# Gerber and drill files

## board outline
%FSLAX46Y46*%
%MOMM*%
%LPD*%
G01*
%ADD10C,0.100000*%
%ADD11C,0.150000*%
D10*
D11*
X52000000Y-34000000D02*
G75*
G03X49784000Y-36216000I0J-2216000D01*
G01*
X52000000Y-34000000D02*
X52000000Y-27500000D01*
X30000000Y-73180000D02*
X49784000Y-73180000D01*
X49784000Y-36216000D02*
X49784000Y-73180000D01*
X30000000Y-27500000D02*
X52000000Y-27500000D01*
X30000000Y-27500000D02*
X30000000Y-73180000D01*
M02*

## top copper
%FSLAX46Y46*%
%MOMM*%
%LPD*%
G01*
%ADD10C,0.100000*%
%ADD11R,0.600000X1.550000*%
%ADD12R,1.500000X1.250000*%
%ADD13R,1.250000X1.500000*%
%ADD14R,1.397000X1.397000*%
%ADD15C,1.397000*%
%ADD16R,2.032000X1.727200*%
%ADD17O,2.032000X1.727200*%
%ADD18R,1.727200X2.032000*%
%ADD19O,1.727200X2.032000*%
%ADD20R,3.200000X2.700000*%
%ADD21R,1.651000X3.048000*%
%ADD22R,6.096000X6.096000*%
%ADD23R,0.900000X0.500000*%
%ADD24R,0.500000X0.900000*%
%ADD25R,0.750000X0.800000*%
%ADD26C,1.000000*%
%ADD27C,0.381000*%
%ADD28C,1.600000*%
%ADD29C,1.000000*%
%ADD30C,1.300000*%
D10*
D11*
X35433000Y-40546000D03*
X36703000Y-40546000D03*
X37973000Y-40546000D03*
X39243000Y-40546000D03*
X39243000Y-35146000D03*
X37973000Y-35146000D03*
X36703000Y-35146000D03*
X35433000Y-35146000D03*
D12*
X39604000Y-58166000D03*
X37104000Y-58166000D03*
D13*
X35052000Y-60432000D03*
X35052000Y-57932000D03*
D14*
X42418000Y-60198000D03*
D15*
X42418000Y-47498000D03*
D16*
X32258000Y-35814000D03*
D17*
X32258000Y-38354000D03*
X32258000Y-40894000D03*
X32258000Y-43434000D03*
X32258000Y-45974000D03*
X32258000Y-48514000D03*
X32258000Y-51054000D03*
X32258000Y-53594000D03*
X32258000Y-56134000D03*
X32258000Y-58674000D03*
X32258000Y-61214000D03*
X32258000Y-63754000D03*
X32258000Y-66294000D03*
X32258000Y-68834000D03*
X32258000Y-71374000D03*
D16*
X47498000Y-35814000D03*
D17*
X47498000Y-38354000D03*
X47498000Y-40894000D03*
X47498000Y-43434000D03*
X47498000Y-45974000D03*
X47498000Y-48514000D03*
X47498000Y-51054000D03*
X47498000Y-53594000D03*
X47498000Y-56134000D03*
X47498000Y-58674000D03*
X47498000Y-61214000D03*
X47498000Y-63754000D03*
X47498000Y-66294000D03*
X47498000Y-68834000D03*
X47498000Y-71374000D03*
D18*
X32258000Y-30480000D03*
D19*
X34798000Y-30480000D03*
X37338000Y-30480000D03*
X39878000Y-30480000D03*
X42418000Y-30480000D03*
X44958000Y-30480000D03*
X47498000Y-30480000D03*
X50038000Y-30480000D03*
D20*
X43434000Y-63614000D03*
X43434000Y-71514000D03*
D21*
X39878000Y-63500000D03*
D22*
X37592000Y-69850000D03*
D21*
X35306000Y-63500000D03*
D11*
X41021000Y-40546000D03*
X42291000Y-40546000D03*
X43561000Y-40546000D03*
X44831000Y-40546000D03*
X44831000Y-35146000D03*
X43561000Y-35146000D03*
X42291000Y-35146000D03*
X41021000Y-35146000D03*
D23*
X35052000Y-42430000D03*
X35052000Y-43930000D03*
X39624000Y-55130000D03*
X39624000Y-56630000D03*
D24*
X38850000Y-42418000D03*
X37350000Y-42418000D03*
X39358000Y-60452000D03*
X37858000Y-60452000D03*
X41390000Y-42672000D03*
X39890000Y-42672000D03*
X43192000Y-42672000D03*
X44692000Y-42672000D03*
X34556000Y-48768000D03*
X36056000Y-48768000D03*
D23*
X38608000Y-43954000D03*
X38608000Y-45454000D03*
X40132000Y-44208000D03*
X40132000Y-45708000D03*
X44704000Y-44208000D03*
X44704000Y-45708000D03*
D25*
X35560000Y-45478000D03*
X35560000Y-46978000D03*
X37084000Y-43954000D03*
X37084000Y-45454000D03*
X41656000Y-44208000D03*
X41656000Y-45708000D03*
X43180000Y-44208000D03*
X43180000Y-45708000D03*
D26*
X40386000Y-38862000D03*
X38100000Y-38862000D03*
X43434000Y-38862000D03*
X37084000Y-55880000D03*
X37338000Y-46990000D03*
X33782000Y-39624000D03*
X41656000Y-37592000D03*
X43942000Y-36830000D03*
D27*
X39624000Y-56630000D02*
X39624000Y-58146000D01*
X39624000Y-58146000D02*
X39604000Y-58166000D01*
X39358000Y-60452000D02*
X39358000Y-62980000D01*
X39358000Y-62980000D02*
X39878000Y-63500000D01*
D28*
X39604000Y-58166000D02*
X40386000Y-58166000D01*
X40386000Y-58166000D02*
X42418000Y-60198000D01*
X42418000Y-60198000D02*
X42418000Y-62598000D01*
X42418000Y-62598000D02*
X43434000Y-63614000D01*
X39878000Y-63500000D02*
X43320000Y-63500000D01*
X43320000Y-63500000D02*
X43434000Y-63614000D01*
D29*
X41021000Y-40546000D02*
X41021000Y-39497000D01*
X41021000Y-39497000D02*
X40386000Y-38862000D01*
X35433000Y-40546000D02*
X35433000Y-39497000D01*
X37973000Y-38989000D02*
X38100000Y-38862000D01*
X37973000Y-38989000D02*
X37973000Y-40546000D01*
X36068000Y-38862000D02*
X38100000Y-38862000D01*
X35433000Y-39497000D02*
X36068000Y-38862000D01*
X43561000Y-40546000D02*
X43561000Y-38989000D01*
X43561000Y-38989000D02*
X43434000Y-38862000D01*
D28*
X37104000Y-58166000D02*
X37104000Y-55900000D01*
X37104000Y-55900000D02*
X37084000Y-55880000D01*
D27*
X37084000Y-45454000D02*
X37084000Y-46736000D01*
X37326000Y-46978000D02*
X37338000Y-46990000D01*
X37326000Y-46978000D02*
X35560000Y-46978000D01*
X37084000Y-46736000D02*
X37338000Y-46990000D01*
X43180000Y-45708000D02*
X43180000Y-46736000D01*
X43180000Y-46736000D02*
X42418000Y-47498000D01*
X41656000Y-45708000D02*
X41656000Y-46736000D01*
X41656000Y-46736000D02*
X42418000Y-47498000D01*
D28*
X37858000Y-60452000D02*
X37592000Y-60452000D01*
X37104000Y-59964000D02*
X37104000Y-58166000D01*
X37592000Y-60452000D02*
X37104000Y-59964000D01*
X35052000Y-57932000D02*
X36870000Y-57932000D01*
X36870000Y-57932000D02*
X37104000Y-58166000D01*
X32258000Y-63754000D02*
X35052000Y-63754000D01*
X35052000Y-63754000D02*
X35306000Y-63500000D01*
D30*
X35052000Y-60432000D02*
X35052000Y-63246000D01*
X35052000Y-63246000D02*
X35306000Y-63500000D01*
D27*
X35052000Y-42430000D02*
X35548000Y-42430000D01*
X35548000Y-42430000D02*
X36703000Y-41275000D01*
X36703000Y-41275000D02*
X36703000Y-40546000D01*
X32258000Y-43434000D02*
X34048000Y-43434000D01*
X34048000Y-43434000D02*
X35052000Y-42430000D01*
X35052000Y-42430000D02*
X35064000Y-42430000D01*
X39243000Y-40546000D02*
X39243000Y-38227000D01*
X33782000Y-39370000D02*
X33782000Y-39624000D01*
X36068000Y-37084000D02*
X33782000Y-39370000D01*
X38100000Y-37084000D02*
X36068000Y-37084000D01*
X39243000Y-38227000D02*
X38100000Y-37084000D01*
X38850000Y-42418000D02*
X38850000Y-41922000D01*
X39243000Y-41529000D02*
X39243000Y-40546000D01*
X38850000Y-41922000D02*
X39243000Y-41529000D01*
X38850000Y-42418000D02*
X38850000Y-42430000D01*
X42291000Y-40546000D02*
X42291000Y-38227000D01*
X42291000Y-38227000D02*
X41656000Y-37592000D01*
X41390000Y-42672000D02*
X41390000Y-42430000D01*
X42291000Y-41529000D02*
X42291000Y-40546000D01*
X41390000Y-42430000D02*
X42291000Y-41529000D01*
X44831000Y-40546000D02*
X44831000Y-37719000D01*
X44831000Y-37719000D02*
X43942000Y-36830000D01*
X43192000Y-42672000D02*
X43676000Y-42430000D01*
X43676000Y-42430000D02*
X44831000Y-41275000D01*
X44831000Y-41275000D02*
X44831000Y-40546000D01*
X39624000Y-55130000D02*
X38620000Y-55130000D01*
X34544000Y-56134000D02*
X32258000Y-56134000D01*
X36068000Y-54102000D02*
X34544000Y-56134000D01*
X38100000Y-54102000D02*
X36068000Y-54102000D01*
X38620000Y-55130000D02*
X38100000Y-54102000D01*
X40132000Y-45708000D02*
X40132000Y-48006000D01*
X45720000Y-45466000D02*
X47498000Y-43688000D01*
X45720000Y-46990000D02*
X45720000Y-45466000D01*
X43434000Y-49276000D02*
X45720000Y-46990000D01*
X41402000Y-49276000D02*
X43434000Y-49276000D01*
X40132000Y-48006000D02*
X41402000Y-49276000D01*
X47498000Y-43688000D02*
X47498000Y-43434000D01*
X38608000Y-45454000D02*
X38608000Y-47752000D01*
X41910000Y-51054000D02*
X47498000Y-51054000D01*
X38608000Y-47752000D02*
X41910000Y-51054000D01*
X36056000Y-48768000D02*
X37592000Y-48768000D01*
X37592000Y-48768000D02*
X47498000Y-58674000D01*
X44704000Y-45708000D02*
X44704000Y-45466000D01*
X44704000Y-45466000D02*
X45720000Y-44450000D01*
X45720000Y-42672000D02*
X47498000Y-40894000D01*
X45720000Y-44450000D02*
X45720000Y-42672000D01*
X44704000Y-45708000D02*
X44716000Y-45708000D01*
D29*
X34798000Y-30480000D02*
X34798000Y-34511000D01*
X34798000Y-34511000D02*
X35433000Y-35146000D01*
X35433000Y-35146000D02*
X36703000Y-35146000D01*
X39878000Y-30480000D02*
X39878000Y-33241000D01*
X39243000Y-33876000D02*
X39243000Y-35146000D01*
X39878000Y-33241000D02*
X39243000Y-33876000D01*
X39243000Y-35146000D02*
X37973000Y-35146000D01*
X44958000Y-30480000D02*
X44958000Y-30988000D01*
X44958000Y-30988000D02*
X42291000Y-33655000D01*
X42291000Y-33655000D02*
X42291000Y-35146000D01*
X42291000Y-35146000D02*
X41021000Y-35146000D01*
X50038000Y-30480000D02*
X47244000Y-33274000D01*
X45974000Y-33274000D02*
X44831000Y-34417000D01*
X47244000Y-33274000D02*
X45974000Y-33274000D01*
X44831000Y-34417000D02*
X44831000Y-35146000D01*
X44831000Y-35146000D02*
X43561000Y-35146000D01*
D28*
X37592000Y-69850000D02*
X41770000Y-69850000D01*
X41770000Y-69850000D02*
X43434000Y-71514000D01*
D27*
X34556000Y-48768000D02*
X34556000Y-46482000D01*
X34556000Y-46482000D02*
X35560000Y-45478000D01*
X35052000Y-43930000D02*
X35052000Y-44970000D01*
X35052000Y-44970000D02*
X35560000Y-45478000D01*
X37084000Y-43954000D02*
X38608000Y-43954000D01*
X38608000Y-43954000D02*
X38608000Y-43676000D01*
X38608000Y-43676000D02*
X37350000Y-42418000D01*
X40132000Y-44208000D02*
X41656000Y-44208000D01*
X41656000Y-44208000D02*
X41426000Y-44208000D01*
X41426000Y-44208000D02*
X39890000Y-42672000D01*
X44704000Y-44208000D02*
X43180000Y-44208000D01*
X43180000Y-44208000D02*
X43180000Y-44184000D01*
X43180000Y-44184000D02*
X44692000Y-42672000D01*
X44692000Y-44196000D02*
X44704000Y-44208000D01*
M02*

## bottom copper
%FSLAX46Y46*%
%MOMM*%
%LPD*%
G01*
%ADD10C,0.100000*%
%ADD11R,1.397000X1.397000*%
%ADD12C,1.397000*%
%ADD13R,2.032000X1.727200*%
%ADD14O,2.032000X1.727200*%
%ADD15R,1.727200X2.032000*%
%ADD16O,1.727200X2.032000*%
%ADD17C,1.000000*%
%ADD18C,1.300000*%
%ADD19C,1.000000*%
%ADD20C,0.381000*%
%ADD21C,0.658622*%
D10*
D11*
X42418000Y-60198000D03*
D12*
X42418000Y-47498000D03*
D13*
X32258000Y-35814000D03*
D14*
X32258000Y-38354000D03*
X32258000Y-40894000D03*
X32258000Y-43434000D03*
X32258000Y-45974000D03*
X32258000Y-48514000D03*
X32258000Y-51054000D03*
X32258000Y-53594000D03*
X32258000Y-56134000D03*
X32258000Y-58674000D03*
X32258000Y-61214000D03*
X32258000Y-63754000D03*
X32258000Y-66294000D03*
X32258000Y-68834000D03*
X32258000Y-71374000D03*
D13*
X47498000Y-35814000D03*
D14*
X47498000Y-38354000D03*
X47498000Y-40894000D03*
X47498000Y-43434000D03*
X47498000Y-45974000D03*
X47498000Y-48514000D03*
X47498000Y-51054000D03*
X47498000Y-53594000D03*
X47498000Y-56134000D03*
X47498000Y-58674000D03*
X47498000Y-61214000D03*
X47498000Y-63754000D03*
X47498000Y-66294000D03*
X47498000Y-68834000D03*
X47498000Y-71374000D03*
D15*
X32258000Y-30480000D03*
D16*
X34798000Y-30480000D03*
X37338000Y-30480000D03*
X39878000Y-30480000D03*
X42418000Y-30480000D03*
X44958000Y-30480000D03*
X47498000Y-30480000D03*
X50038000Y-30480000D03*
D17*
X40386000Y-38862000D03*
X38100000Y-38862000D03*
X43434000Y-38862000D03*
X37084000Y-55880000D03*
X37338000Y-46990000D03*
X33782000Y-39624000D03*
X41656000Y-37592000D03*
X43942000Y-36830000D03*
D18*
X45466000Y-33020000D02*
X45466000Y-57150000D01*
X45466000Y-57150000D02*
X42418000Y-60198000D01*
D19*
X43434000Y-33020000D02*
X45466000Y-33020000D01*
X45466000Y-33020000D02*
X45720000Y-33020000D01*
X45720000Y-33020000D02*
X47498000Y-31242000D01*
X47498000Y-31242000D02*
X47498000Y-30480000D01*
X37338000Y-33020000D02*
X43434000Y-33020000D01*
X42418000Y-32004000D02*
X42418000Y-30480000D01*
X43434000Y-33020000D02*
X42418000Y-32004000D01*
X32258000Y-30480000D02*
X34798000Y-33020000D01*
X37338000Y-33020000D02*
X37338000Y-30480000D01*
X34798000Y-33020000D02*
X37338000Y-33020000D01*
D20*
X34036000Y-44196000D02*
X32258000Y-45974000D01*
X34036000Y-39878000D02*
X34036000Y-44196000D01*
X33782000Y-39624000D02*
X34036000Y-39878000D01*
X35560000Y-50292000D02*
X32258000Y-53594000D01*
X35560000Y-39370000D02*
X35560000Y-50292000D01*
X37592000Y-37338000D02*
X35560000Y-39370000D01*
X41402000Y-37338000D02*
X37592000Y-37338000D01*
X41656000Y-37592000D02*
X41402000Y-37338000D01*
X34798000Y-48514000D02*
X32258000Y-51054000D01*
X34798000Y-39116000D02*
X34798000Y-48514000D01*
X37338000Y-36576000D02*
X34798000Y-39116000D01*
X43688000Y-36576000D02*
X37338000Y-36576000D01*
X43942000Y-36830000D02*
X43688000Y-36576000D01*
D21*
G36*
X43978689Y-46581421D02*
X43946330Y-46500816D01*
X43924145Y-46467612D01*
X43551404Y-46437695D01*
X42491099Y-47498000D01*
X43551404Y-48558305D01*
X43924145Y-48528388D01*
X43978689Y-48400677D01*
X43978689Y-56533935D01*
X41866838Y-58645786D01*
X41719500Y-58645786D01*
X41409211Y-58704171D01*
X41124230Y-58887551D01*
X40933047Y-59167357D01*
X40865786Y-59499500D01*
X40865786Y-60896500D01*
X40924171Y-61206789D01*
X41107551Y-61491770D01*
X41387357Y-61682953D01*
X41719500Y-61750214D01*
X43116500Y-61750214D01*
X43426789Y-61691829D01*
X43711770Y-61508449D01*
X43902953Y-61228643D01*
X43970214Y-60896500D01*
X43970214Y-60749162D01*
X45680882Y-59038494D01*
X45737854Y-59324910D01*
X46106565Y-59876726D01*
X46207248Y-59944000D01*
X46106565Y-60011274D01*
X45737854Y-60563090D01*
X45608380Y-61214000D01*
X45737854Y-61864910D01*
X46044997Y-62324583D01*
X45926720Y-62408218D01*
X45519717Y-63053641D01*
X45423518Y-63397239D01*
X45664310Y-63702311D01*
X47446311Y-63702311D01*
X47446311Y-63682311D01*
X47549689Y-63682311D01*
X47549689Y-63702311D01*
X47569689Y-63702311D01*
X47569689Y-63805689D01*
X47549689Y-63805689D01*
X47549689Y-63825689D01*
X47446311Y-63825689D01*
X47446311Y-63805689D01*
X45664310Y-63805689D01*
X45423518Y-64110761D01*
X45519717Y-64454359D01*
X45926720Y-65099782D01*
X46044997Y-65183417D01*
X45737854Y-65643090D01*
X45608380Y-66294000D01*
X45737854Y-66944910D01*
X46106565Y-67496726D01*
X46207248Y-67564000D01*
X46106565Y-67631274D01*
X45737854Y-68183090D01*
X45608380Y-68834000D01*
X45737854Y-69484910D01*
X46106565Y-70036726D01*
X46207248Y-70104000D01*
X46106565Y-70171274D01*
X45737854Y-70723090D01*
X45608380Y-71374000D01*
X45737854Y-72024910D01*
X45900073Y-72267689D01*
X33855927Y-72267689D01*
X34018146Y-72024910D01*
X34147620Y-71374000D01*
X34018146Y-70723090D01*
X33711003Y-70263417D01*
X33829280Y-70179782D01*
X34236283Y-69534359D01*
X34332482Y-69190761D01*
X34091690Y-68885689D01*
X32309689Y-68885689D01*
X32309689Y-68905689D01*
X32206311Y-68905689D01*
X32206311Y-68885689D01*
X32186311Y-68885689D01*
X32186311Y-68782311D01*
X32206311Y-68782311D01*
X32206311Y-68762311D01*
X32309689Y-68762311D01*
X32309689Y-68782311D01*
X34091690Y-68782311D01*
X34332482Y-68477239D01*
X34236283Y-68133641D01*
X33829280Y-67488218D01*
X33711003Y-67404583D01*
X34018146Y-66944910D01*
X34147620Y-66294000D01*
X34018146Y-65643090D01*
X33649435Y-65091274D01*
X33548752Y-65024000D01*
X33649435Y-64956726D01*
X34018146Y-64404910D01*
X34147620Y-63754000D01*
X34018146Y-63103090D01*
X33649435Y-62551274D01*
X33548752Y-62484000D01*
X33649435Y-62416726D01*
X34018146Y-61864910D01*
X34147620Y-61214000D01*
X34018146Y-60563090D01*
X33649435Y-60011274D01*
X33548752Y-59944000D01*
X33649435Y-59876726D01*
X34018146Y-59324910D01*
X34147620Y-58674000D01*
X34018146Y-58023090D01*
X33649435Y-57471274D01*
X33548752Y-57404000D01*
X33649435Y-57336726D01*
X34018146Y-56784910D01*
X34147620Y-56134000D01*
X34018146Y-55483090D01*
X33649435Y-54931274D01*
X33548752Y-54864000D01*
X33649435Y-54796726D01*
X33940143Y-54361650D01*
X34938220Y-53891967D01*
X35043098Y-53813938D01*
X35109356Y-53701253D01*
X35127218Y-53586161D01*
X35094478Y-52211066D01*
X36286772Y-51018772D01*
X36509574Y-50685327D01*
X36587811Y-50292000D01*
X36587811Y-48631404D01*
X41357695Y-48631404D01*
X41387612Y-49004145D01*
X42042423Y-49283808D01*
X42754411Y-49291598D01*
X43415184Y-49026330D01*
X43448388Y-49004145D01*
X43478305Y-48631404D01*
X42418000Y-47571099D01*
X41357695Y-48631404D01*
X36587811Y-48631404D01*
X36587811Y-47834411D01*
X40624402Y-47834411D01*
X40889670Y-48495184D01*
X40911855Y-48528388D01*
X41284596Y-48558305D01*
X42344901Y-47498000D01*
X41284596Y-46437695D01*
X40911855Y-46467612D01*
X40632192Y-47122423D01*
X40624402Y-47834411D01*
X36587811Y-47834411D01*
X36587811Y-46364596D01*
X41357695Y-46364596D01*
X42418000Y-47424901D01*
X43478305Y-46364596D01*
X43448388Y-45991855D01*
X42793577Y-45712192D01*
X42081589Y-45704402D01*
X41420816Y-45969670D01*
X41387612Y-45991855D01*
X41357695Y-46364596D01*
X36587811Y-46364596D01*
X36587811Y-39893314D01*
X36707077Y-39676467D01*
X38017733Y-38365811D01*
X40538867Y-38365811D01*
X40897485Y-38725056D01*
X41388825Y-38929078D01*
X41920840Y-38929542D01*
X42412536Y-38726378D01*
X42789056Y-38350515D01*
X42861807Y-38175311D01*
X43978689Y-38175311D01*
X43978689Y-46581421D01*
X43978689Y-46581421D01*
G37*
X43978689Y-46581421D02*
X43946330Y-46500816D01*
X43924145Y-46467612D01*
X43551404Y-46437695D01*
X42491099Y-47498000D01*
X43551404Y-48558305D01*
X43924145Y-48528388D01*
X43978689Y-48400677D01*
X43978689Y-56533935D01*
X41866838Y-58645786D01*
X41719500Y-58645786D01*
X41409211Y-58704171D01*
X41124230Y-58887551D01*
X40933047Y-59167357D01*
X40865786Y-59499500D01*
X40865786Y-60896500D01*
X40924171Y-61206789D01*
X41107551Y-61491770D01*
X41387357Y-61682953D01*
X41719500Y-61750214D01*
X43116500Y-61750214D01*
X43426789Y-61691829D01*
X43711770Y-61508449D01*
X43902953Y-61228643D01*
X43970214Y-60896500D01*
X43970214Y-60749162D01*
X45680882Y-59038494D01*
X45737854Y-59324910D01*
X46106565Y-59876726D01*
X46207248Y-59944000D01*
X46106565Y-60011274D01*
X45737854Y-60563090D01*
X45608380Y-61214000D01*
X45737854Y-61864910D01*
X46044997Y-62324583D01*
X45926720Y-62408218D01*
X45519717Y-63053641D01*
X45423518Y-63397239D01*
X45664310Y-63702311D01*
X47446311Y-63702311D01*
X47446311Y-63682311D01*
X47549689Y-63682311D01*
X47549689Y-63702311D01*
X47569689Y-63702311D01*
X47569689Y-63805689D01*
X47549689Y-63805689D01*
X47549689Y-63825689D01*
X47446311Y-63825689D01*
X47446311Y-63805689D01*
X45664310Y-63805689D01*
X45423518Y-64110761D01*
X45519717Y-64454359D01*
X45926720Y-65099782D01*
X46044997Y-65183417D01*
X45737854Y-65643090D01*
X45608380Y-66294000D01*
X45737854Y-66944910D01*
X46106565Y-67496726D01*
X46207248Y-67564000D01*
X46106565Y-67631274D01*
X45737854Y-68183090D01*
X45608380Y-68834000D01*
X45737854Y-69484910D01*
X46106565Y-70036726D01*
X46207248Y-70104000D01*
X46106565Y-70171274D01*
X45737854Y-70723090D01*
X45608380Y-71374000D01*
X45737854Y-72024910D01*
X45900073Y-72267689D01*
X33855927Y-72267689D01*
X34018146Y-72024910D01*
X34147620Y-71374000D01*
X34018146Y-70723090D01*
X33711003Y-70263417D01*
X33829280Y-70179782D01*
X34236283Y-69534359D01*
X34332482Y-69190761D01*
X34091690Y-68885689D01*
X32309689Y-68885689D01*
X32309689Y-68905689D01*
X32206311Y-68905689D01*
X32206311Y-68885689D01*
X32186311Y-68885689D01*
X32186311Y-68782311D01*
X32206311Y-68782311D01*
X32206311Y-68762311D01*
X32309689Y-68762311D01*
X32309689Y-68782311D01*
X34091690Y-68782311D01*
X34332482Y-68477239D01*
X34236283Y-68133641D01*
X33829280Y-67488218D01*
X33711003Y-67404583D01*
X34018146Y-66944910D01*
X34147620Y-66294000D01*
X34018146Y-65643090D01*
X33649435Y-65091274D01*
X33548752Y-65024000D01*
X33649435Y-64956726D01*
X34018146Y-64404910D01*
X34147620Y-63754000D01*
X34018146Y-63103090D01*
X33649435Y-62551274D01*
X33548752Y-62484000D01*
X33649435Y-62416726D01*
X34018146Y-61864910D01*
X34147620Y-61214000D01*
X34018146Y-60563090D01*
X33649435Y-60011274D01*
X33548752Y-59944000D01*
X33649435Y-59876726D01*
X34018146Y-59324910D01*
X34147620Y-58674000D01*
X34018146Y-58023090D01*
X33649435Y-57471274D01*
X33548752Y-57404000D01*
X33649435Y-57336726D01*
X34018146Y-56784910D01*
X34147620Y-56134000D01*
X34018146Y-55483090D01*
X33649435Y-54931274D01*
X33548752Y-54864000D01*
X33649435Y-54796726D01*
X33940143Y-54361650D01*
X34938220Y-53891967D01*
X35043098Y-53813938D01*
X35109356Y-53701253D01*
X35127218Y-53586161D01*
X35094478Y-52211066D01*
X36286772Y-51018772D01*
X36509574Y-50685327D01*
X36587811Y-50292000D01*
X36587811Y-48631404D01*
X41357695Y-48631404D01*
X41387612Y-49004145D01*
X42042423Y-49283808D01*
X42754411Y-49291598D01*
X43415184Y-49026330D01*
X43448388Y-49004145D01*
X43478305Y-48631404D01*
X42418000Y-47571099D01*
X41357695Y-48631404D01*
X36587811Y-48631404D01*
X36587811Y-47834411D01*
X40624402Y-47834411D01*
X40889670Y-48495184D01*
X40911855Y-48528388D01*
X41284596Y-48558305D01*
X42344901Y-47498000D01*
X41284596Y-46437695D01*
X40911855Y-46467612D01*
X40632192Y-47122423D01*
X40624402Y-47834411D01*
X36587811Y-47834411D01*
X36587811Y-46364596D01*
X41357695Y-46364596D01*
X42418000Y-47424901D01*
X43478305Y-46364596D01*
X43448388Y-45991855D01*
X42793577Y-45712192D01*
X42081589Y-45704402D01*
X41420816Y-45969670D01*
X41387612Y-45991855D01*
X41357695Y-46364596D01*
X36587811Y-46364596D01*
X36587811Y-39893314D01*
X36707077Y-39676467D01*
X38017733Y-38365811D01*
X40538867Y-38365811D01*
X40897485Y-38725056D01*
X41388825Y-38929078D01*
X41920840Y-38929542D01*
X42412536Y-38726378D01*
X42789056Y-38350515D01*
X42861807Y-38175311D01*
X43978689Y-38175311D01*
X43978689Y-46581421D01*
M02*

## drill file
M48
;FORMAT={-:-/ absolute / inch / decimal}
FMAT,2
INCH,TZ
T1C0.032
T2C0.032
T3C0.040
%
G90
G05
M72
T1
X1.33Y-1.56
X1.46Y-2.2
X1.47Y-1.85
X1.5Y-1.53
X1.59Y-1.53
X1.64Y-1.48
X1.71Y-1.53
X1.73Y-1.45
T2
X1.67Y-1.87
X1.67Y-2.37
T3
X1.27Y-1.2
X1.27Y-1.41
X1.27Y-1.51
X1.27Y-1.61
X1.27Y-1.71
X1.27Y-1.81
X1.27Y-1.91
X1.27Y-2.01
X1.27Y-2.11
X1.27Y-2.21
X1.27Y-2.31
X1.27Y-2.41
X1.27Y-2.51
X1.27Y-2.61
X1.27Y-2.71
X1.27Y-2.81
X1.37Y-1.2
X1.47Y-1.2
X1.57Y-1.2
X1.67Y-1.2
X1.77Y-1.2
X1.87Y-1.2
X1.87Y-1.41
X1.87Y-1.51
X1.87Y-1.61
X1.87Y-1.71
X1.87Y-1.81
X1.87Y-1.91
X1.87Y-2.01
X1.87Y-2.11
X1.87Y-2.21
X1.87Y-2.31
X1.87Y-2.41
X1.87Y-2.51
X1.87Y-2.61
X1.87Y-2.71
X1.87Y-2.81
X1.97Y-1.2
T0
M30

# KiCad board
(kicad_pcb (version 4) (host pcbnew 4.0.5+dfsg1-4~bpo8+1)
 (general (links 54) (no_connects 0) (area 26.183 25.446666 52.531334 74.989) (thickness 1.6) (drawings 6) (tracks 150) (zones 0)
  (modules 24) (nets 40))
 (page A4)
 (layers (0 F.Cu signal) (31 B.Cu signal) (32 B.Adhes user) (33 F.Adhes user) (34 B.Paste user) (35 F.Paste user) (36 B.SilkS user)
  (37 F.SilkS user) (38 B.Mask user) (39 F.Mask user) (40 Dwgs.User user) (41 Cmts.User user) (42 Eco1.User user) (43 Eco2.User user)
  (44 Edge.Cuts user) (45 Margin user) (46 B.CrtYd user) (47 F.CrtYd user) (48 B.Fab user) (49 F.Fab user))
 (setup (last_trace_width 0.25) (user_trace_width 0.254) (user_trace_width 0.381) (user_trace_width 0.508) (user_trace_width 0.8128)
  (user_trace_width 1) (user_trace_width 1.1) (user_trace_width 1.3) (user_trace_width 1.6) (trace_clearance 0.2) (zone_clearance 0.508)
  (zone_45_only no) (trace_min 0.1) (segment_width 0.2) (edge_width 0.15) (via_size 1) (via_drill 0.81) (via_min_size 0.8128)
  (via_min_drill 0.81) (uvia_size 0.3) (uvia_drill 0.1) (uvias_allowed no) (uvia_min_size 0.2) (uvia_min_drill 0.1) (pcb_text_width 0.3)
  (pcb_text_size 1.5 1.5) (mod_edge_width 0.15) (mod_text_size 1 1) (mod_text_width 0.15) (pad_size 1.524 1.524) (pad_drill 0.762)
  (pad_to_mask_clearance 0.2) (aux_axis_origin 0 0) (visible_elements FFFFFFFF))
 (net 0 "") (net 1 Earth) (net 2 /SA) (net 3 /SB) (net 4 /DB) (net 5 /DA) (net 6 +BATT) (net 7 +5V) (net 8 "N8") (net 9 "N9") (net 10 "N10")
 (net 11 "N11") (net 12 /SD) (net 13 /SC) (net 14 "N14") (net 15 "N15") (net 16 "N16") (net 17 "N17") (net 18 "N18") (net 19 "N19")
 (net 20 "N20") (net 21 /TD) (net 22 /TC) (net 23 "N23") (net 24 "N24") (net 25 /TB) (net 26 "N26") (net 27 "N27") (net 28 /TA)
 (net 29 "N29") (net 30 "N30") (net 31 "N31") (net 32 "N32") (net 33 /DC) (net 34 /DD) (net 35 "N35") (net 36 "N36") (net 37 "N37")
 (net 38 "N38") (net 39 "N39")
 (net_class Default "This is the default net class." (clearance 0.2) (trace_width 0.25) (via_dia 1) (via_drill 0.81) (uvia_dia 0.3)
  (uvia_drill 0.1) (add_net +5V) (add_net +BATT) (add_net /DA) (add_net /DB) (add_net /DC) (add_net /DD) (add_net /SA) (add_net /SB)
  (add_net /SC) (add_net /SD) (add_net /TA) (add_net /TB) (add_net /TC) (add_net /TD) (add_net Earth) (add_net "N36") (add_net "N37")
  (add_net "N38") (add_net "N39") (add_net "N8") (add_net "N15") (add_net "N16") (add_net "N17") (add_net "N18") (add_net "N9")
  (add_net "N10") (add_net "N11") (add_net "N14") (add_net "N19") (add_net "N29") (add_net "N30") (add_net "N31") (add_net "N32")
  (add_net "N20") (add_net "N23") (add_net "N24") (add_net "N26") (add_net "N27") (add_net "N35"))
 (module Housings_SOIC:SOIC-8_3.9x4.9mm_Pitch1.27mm (layer F.Cu) (at 37.338 37.846 90)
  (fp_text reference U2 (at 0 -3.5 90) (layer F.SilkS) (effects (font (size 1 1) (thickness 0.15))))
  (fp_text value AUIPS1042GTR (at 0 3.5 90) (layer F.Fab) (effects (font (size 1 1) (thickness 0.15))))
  (pad 1 smd rect (at -2.7 -1.905 90) (size 1.55 0.6) (layers F.Cu F.Paste F.Mask) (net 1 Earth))
  (pad 2 smd rect (at -2.7 -0.635 90) (size 1.55 0.6) (layers F.Cu F.Paste F.Mask) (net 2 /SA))
  (pad 3 smd rect (at -2.7 0.635 90) (size 1.55 0.6) (layers F.Cu F.Paste F.Mask) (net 1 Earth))
  (pad 4 smd rect (at -2.7 1.905 90) (size 1.55 0.6) (layers F.Cu F.Paste F.Mask) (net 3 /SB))
  (pad 5 smd rect (at 2.7 1.905 90) (size 1.55 0.6) (layers F.Cu F.Paste F.Mask) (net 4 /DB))
  (pad 6 smd rect (at 2.7 0.635 90) (size 1.55 0.6) (layers F.Cu F.Paste F.Mask) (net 4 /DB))
  (pad 7 smd rect (at 2.7 -0.635 90) (size 1.55 0.6) (layers F.Cu F.Paste F.Mask) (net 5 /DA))
  (pad 8 smd rect (at 2.7 -1.905 90) (size 1.55 0.6) (layers F.Cu F.Paste F.Mask) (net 5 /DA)))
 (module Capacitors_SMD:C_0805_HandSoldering (layer F.Cu) (at 38.354 58.166 180)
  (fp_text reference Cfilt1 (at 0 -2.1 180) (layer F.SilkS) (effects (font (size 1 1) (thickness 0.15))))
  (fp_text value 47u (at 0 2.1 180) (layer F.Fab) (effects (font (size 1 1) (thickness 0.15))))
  (pad 1 smd rect (at -1.25 0 180) (size 1.5 1.25) (layers F.Cu F.Paste F.Mask) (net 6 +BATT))
  (pad 2 smd rect (at 1.25 0 180) (size 1.5 1.25) (layers F.Cu F.Paste F.Mask) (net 1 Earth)))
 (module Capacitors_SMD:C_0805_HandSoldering (layer F.Cu) (at 35.052 59.182 90)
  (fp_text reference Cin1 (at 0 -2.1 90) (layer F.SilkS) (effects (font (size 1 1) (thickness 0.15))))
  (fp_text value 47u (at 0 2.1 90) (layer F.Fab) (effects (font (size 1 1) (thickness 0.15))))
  (pad 1 smd rect (at -1.25 0 90) (size 1.5 1.25) (layers F.Cu F.Paste F.Mask) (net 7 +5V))
  (pad 2 smd rect (at 1.25 0 90) (size 1.5 1.25) (layers F.Cu F.Paste F.Mask) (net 1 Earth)))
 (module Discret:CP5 (layer F.Cu) (at 42.418 53.848 90)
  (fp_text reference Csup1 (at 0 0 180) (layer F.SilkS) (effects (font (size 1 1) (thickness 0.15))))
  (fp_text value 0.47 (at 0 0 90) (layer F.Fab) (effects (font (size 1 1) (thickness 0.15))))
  (pad 1 thru_hole rect (at -6.35 0 90) (size 1.397 1.397) (drill 0.8128) (layers *.Cu *.Mask) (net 6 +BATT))
  (pad 2 thru_hole circle (at 6.35 0 90) (size 1.397 1.397) (drill 0.8128) (layers *.Cu *.Mask) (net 1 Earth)))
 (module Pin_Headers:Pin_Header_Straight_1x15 (layer F.Cu) (at 32.258 35.814)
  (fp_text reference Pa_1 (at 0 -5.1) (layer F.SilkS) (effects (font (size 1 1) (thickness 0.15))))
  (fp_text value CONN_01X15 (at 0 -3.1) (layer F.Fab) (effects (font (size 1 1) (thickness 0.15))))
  (pad 1 thru_hole rect (at 0 0) (size 2.032 1.7272) (drill 1.016) (layers *.Cu *.Mask) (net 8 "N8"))
  (pad 2 thru_hole oval (at 0 2.54) (size 2.032 1.7272) (drill 1.016) (layers *.Cu *.Mask) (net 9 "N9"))
  (pad 3 thru_hole oval (at 0 5.08) (size 2.032 1.7272) (drill 1.016) (layers *.Cu *.Mask) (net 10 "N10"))
  (pad 4 thru_hole oval (at 0 7.62) (size 2.032 1.7272) (drill 1.016) (layers *.Cu *.Mask) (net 2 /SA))
  (pad 5 thru_hole oval (at 0 10.16) (size 2.032 1.7272) (drill 1.016) (layers *.Cu *.Mask) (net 3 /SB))
  (pad 6 thru_hole oval (at 0 12.7) (size 2.032 1.7272) (drill 1.016) (layers *.Cu *.Mask) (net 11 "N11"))
  (pad 7 thru_hole oval (at 0 15.24) (size 2.032 1.7272) (drill 1.016) (layers *.Cu *.Mask) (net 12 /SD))
  (pad 8 thru_hole oval (at 0 17.78) (size 2.032 1.7272) (drill 1.016) (layers *.Cu *.Mask) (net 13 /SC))
  (pad 9 thru_hole oval (at 0 20.32) (size 2.032 1.7272) (drill 1.016) (layers *.Cu *.Mask) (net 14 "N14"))
  (pad 10 thru_hole oval (at 0 22.86) (size 2.032 1.7272) (drill 1.016) (layers *.Cu *.Mask) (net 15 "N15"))
  (pad 11 thru_hole oval (at 0 25.4) (size 2.032 1.7272) (drill 1.016) (layers *.Cu *.Mask) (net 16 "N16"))
  (pad 12 thru_hole oval (at 0 27.94) (size 2.032 1.7272) (drill 1.016) (layers *.Cu *.Mask) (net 7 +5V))
  (pad 13 thru_hole oval (at 0 30.48) (size 2.032 1.7272) (drill 1.016) (layers *.Cu *.Mask) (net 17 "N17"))
  (pad 14 thru_hole oval (at 0 33.02) (size 2.032 1.7272) (drill 1.016) (layers *.Cu *.Mask) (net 1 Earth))
  (pad 15 thru_hole oval (at 0 35.56) (size 2.032 1.7272) (drill 1.016) (layers *.Cu *.Mask) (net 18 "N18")))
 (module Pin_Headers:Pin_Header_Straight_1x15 (layer F.Cu) (at 47.498 35.814)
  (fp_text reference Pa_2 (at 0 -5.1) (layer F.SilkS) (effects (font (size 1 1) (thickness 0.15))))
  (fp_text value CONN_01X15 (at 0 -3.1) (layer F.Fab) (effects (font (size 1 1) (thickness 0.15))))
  (pad 1 thru_hole rect (at 0 0) (size 2.032 1.7272) (drill 1.016) (layers *.Cu *.Mask) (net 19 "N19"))
  (pad 2 thru_hole oval (at 0 2.54) (size 2.032 1.7272) (drill 1.016) (layers *.Cu *.Mask) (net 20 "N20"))
  (pad 3 thru_hole oval (at 0 5.08) (size 2.032 1.7272) (drill 1.016) (layers *.Cu *.Mask) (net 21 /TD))
  (pad 4 thru_hole oval (at 0 7.62) (size 2.032 1.7272) (drill 1.016) (layers *.Cu *.Mask) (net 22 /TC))
  (pad 5 thru_hole oval (at 0 10.16) (size 2.032 1.7272) (drill 1.016) (layers *.Cu *.Mask) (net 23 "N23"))
  (pad 6 thru_hole oval (at 0 12.7) (size 2.032 1.7272) (drill 1.016) (layers *.Cu *.Mask) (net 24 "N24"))
  (pad 7 thru_hole oval (at 0 15.24) (size 2.032 1.7272) (drill 1.016) (layers *.Cu *.Mask) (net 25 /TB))
  (pad 8 thru_hole oval (at 0 17.78) (size 2.032 1.7272) (drill 1.016) (layers *.Cu *.Mask) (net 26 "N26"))
  (pad 9 thru_hole oval (at 0 20.32) (size 2.032 1.7272) (drill 1.016) (layers *.Cu *.Mask) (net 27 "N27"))
  (pad 10 thru_hole oval (at 0 22.86) (size 2.032 1.7272) (drill 1.016) (layers *.Cu *.Mask) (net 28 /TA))
  (pad 11 thru_hole oval (at 0 25.4) (size 2.032 1.7272) (drill 1.016) (layers *.Cu *.Mask) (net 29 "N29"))
  (pad 12 thru_hole oval (at 0 27.94) (size 2.032 1.7272) (drill 1.016) (layers *.Cu *.Mask) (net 1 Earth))
  (pad 13 thru_hole oval (at 0 30.48) (size 2.032 1.7272) (drill 1.016) (layers *.Cu *.Mask) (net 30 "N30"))
  (pad 14 thru_hole oval (at 0 33.02) (size 2.032 1.7272) (drill 1.016) (layers *.Cu *.Mask) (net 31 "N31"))
  (pad 15 thru_hole oval (at 0 35.56) (size 2.032 1.7272) (drill 1.016) (layers *.Cu *.Mask) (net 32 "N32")))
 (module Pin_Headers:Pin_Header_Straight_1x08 (layer F.Cu) (at 32.258 30.48 90)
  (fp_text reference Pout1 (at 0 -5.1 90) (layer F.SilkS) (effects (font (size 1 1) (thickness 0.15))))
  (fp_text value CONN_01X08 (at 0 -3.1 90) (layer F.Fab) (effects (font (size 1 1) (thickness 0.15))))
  (pad 1 thru_hole rect (at 0 0 90) (size 2.032 1.7272) (drill 1.016) (layers *.Cu *.Mask) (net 6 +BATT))
  (pad 2 thru_hole oval (at 0 2.54 90) (size 2.032 1.7272) (drill 1.016) (layers *.Cu *.Mask) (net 5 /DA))
  (pad 3 thru_hole oval (at 0 5.08 90) (size 2.032 1.7272) (drill 1.016) (layers *.Cu *.Mask) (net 6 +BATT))
  (pad 4 thru_hole oval (at 0 7.62 90) (size 2.032 1.7272) (drill 1.016) (layers *.Cu *.Mask) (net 4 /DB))
  (pad 5 thru_hole oval (at 0 10.16 90) (size 2.032 1.7272) (drill 1.016) (layers *.Cu *.Mask) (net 6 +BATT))
  (pad 6 thru_hole oval (at 0 12.7 90) (size 2.032 1.7272) (drill 1.016) (layers *.Cu *.Mask) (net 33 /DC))
  (pad 7 thru_hole oval (at 0 15.24 90) (size 2.032 1.7272) (drill 1.016) (layers *.Cu *.Mask) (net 6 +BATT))
  (pad 8 thru_hole oval (at 0 17.78 90) (size 2.032 1.7272) (drill 1.016) (layers *.Cu *.Mask) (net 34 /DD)))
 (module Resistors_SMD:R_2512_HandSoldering (layer F.Cu) (at 43.434 67.564 270)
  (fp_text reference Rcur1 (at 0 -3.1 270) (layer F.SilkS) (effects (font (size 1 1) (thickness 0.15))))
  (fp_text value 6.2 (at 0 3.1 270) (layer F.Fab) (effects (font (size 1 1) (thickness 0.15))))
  (pad 1 smd rect (at -3.95 0 270) (size 2.7 3.2) (layers F.Cu F.Paste F.Mask) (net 6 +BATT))
  (pad 2 smd rect (at 3.95 0 270) (size 2.7 3.2) (layers F.Cu F.Paste F.Mask) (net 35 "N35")))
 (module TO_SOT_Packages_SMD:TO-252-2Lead (layer F.Cu) (at 37.592 63.5 180)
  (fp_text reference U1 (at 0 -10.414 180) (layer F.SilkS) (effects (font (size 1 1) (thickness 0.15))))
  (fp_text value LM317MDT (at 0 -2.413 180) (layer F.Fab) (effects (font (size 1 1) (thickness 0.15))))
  (pad 1 smd rect (at -2.286 0 180) (size 1.651 3.048) (layers F.Cu F.Paste F.Mask) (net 6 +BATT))
  (pad 2 smd rect (at 0 -6.35 180) (size 6.096 6.096) (layers F.Cu F.Paste F.Mask) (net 35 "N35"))
  (pad 3 smd rect (at 2.286 0 180) (size 1.651 3.048) (layers F.Cu F.Paste F.Mask) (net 7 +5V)))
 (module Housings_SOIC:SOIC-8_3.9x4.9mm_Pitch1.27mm (layer F.Cu) (at 42.926 37.846 90)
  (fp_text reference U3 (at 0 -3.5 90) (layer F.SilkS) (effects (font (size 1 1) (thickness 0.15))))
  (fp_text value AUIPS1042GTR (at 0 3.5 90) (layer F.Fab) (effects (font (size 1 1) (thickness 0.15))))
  (pad 1 smd rect (at -2.7 -1.905 90) (size 1.55 0.6) (layers F.Cu F.Paste F.Mask) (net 1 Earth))
  (pad 2 smd rect (at -2.7 -0.635 90) (size 1.55 0.6) (layers F.Cu F.Paste F.Mask) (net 13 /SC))
  (pad 3 smd rect (at -2.7 0.635 90) (size 1.55 0.6) (layers F.Cu F.Paste F.Mask) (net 1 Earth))
  (pad 4 smd rect (at -2.7 1.905 90) (size 1.55 0.6) (layers F.Cu F.Paste F.Mask) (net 12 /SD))
  (pad 5 smd rect (at 2.7 1.905 90) (size 1.55 0.6) (layers F.Cu F.Paste F.Mask) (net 34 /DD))
  (pad 6 smd rect (at 2.7 0.635 90) (size 1.55 0.6) (layers F.Cu F.Paste F.Mask) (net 34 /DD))
  (pad 7 smd rect (at 2.7 -0.635 90) (size 1.55 0.6) (layers F.Cu F.Paste F.Mask) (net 33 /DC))
  (pad 8 smd rect (at 2.7 -1.905 90) (size 1.55 0.6) (layers F.Cu F.Paste F.Mask) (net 33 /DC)))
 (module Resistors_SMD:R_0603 (layer F.Cu) (at 35.052 43.18 270)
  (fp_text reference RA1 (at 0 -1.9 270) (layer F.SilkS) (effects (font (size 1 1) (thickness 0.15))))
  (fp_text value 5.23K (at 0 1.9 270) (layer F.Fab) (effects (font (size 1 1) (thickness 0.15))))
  (pad 1 smd rect (at -0.75 0 270) (size 0.5 0.9) (layers F.Cu F.Paste F.Mask) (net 2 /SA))
  (pad 2 smd rect (at 0.75 0 270) (size 0.5 0.9) (layers F.Cu F.Paste F.Mask) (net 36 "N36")))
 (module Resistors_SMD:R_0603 (layer F.Cu) (at 39.624 55.88 270)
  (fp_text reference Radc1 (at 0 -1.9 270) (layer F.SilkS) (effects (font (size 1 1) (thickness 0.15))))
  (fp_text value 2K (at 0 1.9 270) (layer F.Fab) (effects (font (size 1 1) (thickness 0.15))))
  (pad 1 smd rect (at -0.75 0 270) (size 0.5 0.9) (layers F.Cu F.Paste F.Mask) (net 14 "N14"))
  (pad 2 smd rect (at 0.75 0 270) (size 0.5 0.9) (layers F.Cu F.Paste F.Mask) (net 6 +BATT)))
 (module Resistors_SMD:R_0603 (layer F.Cu) (at 38.1 42.418 180)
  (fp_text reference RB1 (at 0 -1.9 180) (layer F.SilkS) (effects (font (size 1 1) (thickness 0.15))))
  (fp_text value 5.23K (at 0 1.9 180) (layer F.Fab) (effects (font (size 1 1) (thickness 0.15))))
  (pad 1 smd rect (at -0.75 0 180) (size 0.5 0.9) (layers F.Cu F.Paste F.Mask) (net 3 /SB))
  (pad 2 smd rect (at 0.75 0 180) (size 0.5 0.9) (layers F.Cu F.Paste F.Mask) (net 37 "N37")))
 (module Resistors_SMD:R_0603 (layer F.Cu) (at 38.608 60.452 180)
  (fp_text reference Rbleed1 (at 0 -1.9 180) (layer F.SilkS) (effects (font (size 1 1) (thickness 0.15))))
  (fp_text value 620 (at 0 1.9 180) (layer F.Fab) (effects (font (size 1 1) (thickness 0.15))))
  (pad 1 smd rect (at -0.75 0 180) (size 0.5 0.9) (layers F.Cu F.Paste F.Mask) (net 6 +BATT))
  (pad 2 smd rect (at 0.75 0 180) (size 0.5 0.9) (layers F.Cu F.Paste F.Mask) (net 1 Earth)))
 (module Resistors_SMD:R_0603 (layer F.Cu) (at 40.64 42.672 180)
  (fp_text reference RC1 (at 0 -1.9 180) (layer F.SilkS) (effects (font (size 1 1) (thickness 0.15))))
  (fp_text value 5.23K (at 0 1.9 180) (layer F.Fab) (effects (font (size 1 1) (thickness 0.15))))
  (pad 1 smd rect (at -0.75 0 180) (size 0.5 0.9) (layers F.Cu F.Paste F.Mask) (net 13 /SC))
  (pad 2 smd rect (at 0.75 0 180) (size 0.5 0.9) (layers F.Cu F.Paste F.Mask) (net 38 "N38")))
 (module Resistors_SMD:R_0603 (layer F.Cu) (at 43.942 42.672)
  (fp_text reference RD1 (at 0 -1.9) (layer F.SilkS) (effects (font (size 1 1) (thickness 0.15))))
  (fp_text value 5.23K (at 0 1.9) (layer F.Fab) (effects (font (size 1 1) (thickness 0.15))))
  (pad 1 smd rect (at -0.75 0) (size 0.5 0.9) (layers F.Cu F.Paste F.Mask) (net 12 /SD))
  (pad 2 smd rect (at 0.75 0) (size 0.5 0.9) (layers F.Cu F.Paste F.Mask) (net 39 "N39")))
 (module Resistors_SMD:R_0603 (layer F.Cu) (at 35.306 48.768)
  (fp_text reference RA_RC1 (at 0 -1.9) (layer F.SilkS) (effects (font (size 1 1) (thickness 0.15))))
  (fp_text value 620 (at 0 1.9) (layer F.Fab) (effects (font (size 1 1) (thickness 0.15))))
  (pad 1 smd rect (at -0.75 0) (size 0.5 0.9) (layers F.Cu F.Paste F.Mask) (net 36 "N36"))
  (pad 2 smd rect (at 0.75 0) (size 0.5 0.9) (layers F.Cu F.Paste F.Mask) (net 28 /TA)))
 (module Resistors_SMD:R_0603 (layer F.Cu) (at 38.608 44.704 270)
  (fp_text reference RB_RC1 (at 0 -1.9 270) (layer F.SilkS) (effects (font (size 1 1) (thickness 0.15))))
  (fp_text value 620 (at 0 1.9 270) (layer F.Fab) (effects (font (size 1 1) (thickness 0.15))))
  (pad 1 smd rect (at -0.75 0 270) (size 0.5 0.9) (layers F.Cu F.Paste F.Mask) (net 37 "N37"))
  (pad 2 smd rect (at 0.75 0 270) (size 0.5 0.9) (layers F.Cu F.Paste F.Mask) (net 25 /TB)))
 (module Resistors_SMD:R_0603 (layer F.Cu) (at 40.132 44.958 270)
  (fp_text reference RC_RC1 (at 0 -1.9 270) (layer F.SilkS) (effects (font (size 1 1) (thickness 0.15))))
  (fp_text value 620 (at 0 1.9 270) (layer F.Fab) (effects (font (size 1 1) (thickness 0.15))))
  (pad 1 smd rect (at -0.75 0 270) (size 0.5 0.9) (layers F.Cu F.Paste F.Mask) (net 38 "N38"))
  (pad 2 smd rect (at 0.75 0 270) (size 0.5 0.9) (layers F.Cu F.Paste F.Mask) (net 22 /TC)))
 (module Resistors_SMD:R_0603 (layer F.Cu) (at 44.704 44.958 270)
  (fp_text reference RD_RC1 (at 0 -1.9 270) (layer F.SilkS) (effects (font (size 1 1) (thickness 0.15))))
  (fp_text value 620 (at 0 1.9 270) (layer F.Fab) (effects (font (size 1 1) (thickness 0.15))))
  (pad 1 smd rect (at -0.75 0 270) (size 0.5 0.9) (layers F.Cu F.Paste F.Mask) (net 39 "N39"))
  (pad 2 smd rect (at 0.75 0 270) (size 0.5 0.9) (layers F.Cu F.Paste F.Mask) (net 21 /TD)))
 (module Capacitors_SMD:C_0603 (layer F.Cu) (at 35.56 46.228 270)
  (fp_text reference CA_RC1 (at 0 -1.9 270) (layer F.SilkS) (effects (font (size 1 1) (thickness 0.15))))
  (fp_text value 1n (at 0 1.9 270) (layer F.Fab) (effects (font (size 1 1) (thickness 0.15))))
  (pad 1 smd rect (at -0.75 0 270) (size 0.8 0.75) (layers F.Cu F.Paste F.Mask) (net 36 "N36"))
  (pad 2 smd rect (at 0.75 0 270) (size 0.8 0.75) (layers F.Cu F.Paste F.Mask) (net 1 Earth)))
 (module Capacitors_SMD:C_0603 (layer F.Cu) (at 37.084 44.704 270)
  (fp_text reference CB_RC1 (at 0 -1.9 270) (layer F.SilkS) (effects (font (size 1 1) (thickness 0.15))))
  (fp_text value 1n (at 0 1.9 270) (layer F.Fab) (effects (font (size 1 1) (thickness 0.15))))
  (pad 1 smd rect (at -0.75 0 270) (size 0.8 0.75) (layers F.Cu F.Paste F.Mask) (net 37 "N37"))
  (pad 2 smd rect (at 0.75 0 270) (size 0.8 0.75) (layers F.Cu F.Paste F.Mask) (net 1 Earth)))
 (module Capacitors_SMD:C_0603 (layer F.Cu) (at 41.656 44.958 270)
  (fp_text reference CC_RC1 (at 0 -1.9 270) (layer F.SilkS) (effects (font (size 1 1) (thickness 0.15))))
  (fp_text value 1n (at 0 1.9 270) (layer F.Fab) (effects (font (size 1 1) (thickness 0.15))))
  (pad 1 smd rect (at -0.75 0 270) (size 0.8 0.75) (layers F.Cu F.Paste F.Mask) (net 38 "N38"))
  (pad 2 smd rect (at 0.75 0 270) (size 0.8 0.75) (layers F.Cu F.Paste F.Mask) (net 1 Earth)))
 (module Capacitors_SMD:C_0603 (layer F.Cu) (at 43.18 44.958 270)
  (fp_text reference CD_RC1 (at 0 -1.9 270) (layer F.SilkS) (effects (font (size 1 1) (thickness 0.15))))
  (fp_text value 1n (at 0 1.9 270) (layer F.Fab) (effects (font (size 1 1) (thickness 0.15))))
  (pad 1 smd rect (at -0.75 0 270) (size 0.8 0.75) (layers F.Cu F.Paste F.Mask) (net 39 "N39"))
  (pad 2 smd rect (at 0.75 0 270) (size 0.8 0.75) (layers F.Cu F.Paste F.Mask) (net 1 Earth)))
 (gr_arc (start 52 36.216) (end 49.784 36.216) (angle 90) (layer Edge.Cuts) (width 0.15))
 (gr_line (start 52 34) (end 52 27.5) (angle 90) (layer Edge.Cuts) (width 0.15))
 (gr_line (start 30 73.18) (end 49.784 73.18) (angle 90) (layer Edge.Cuts) (width 0.15))
 (gr_line (start 49.784 36.216) (end 49.784 73.18) (angle 90) (layer Edge.Cuts) (width 0.15))
 (gr_line (start 30 27.5) (end 52 27.5) (angle 90) (layer Edge.Cuts) (width 0.15))
 (gr_line (start 30 27.5) (end 30 73.18) (angle 90) (layer Edge.Cuts) (width 0.15))
 (segment (start 39.624 56.63) (end 39.624 58.146) (width 0.381) (layer F.Cu) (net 6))
 (segment (start 39.624 58.146) (end 39.604 58.166) (width 0.381) (layer F.Cu) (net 6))
 (segment (start 39.358 60.452) (end 39.358 62.98) (width 0.381) (layer F.Cu) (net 6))
 (segment (start 39.358 62.98) (end 39.878 63.5) (width 0.381) (layer F.Cu) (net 6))
 (segment (start 39.604 58.166) (end 40.386 58.166) (width 1.6) (layer F.Cu) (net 6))
 (segment (start 40.386 58.166) (end 42.418 60.198) (width 1.6) (layer F.Cu) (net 6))
 (segment (start 42.418 60.198) (end 42.418 62.598) (width 1.6) (layer F.Cu) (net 6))
 (segment (start 42.418 62.598) (end 43.434 63.614) (width 1.6) (layer F.Cu) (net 6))
 (segment (start 39.878 63.5) (end 43.32 63.5) (width 1.6) (layer F.Cu) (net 6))
 (segment (start 43.32 63.5) (end 43.434 63.614) (width 1.6) (layer F.Cu) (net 6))
 (segment (start 45.466 33.02) (end 45.466 57.15) (width 1.3) (layer B.Cu) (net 6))
 (segment (start 45.466 57.15) (end 42.418 60.198) (width 1.3) (layer B.Cu) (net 6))
 (segment (start 43.434 33.02) (end 45.466 33.02) (width 1) (layer B.Cu) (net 6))
 (segment (start 45.466 33.02) (end 45.72 33.02) (width 1) (layer B.Cu) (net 6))
 (segment (start 45.72 33.02) (end 47.498 31.242) (width 1) (layer B.Cu) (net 6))
 (segment (start 47.498 31.242) (end 47.498 30.48) (width 1) (layer B.Cu) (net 6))
 (segment (start 37.338 33.02) (end 43.434 33.02) (width 1) (layer B.Cu) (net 6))
 (segment (start 42.418 32.004) (end 42.418 30.48) (width 1) (layer B.Cu) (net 6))
 (segment (start 43.434 33.02) (end 42.418 32.004) (width 1) (layer B.Cu) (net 6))
 (segment (start 32.258 30.48) (end 34.798 33.02) (width 1) (layer B.Cu) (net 6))
 (segment (start 37.338 33.02) (end 37.338 30.48) (width 1) (layer B.Cu) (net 6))
 (segment (start 34.798 33.02) (end 37.338 33.02) (width 1) (layer B.Cu) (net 6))
 (segment (start 41.021 40.546) (end 41.021 39.497) (width 1) (layer F.Cu) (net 1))
 (via (at 40.386 38.862) (size 1) (drill 0.81) (layers F.Cu B.Cu) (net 1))
 (segment (start 41.021 39.497) (end 40.386 38.862) (width 1) (layer F.Cu) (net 1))
 (segment (start 35.433 40.546) (end 35.433 39.497) (width 1) (layer F.Cu) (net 1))
 (segment (start 37.973 38.989) (end 38.1 38.862) (width 1) (layer F.Cu) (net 1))
 (via (at 38.1 38.862) (size 1) (drill 0.81) (layers F.Cu B.Cu) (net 1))
 (segment (start 37.973 38.989) (end 37.973 40.546) (width 1) (layer F.Cu) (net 1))
 (segment (start 36.068 38.862) (end 38.1 38.862) (width 1) (layer F.Cu) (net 1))
 (segment (start 35.433 39.497) (end 36.068 38.862) (width 1) (layer F.Cu) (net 1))
 (segment (start 43.561 40.546) (end 43.561 38.989) (width 1) (layer F.Cu) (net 1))
 (via (at 43.434 38.862) (size 1) (drill 0.81) (layers F.Cu B.Cu) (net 1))
 (segment (start 43.561 38.989) (end 43.434 38.862) (width 1) (layer F.Cu) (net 1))
 (segment (start 37.104 58.166) (end 37.104 55.9) (width 1.6) (layer F.Cu) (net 1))
 (via (at 37.084 55.88) (size 1) (drill 0.81) (layers F.Cu B.Cu) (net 1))
 (segment (start 37.104 55.9) (end 37.084 55.88) (width 1.6) (layer F.Cu) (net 1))
 (segment (start 37.084 45.454) (end 37.084 46.736) (width 0.381) (layer F.Cu) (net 1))
 (segment (start 37.326 46.978) (end 37.338 46.99) (width 0.381) (layer F.Cu) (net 1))
 (via (at 37.338 46.99) (size 1) (drill 0.81) (layers F.Cu B.Cu) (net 1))
 (segment (start 37.326 46.978) (end 35.56 46.978) (width 0.381) (layer F.Cu) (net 1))
 (segment (start 37.084 46.736) (end 37.338 46.99) (width 0.381) (layer F.Cu) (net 1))
 (segment (start 43.18 45.708) (end 43.18 46.736) (width 0.381) (layer F.Cu) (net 1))
 (segment (start 43.18 46.736) (end 42.418 47.498) (width 0.381) (layer F.Cu) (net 1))
 (segment (start 41.656 45.708) (end 41.656 46.736) (width 0.381) (layer F.Cu) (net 1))
 (segment (start 41.656 46.736) (end 42.418 47.498) (width 0.381) (layer F.Cu) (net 1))
 (segment (start 37.858 60.452) (end 37.592 60.452) (width 1.6) (layer F.Cu) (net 1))
 (segment (start 37.104 59.964) (end 37.104 58.166) (width 1.6) (layer F.Cu) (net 1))
 (segment (start 37.592 60.452) (end 37.104 59.964) (width 1.6) (layer F.Cu) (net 1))
 (segment (start 35.052 57.932) (end 36.87 57.932) (width 1.6) (layer F.Cu) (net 1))
 (segment (start 36.87 57.932) (end 37.104 58.166) (width 1.6) (layer F.Cu) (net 1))
 (segment (start 32.258 63.754) (end 35.052 63.754) (width 1.6) (layer F.Cu) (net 7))
 (segment (start 35.052 63.754) (end 35.306 63.5) (width 1.6) (layer F.Cu) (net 7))
 (segment (start 35.052 60.432) (end 35.052 63.246) (width 1.3) (layer F.Cu) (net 7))
 (segment (start 35.052 63.246) (end 35.306 63.5) (width 1.3) (layer F.Cu) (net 7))
 (segment (start 35.052 42.43) (end 35.548 42.43) (width 0.381) (layer F.Cu) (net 2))
 (segment (start 35.548 42.43) (end 36.703 41.275) (width 0.381) (layer F.Cu) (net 2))
 (segment (start 36.703 41.275) (end 36.703 40.546) (width 0.381) (layer F.Cu) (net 2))
 (segment (start 32.258 43.434) (end 34.048 43.434) (width 0.381) (layer F.Cu) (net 2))
 (segment (start 34.048 43.434) (end 35.052 42.43) (width 0.381) (layer F.Cu) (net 2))
 (segment (start 35.052 42.43) (end 35.064 42.43) (width 0.381) (layer F.Cu) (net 2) (status 30))
 (segment (start 39.243 40.546) (end 39.243 38.227) (width 0.381) (layer F.Cu) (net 3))
 (segment (start 34.036 44.196) (end 32.258 45.974) (width 0.381) (layer B.Cu) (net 3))
 (segment (start 34.036 39.878) (end 34.036 44.196) (width 0.381) (layer B.Cu) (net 3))
 (segment (start 33.782 39.624) (end 34.036 39.878) (width 0.381) (layer B.Cu) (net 3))
 (via (at 33.782 39.624) (size 1) (drill 0.81) (layers F.Cu B.Cu) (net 3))
 (segment (start 33.782 39.37) (end 33.782 39.624) (width 0.381) (layer F.Cu) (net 3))
 (segment (start 36.068 37.084) (end 33.782 39.37) (width 0.381) (layer F.Cu) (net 3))
 (segment (start 38.1 37.084) (end 36.068 37.084) (width 0.381) (layer F.Cu) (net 3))
 (segment (start 39.243 38.227) (end 38.1 37.084) (width 0.381) (layer F.Cu) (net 3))
 (segment (start 38.85 42.418) (end 38.85 41.922) (width 0.381) (layer F.Cu) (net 3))
 (segment (start 39.243 41.529) (end 39.243 40.546) (width 0.381) (layer F.Cu) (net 3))
 (segment (start 38.85 41.922) (end 39.243 41.529) (width 0.381) (layer F.Cu) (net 3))
 (segment (start 38.85 42.418) (end 38.85 42.43) (width 0.381) (layer F.Cu) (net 3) (status 30))
 (segment (start 42.291 40.546) (end 42.291 38.227) (width 0.381) (layer F.Cu) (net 13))
 (segment (start 35.56 50.292) (end 32.258 53.594) (width 0.381) (layer B.Cu) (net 13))
 (segment (start 35.56 39.37) (end 35.56 50.292) (width 0.381) (layer B.Cu) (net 13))
 (segment (start 37.592 37.338) (end 35.56 39.37) (width 0.381) (layer B.Cu) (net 13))
 (segment (start 41.402 37.338) (end 37.592 37.338) (width 0.381) (layer B.Cu) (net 13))
 (segment (start 41.656 37.592) (end 41.402 37.338) (width 0.381) (layer B.Cu) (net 13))
 (via (at 41.656 37.592) (size 1) (drill 0.81) (layers F.Cu B.Cu) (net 13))
 (segment (start 42.291 38.227) (end 41.656 37.592) (width 0.381) (layer F.Cu) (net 13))
 (segment (start 41.39 42.672) (end 41.39 42.43) (width 0.381) (layer F.Cu) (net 13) (status 10))
 (segment (start 42.291 41.529) (end 42.291 40.546) (width 0.381) (layer F.Cu) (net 13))
 (segment (start 41.39 42.43) (end 42.291 41.529) (width 0.381) (layer F.Cu) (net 13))
 (segment (start 44.831 40.546) (end 44.831 37.719) (width 0.381) (layer F.Cu) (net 12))
 (segment (start 34.798 48.514) (end 32.258 51.054) (width 0.381) (layer B.Cu) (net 12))
 (segment (start 34.798 39.116) (end 34.798 48.514) (width 0.381) (layer B.Cu) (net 12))
 (segment (start 37.338 36.576) (end 34.798 39.116) (width 0.381) (layer B.Cu) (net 12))
 (segment (start 43.688 36.576) (end 37.338 36.576) (width 0.381) (layer B.Cu) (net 12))
 (segment (start 43.942 36.83) (end 43.688 36.576) (width 0.381) (layer B.Cu) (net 12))
 (via (at 43.942 36.83) (size 1) (drill 0.81) (layers F.Cu B.Cu) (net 12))
 (segment (start 44.831 37.719) (end 43.942 36.83) (width 0.381) (layer F.Cu) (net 12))
 (segment (start 43.192 42.672) (end 43.676 42.43) (width 0.381) (layer F.Cu) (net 12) (status 10))
 (segment (start 43.676 42.43) (end 44.831 41.275) (width 0.381) (layer F.Cu) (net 12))
 (segment (start 44.831 41.275) (end 44.831 40.546) (width 0.381) (layer F.Cu) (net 12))
 (segment (start 39.624 55.13) (end 38.62 55.13) (width 0.381) (layer F.Cu) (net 14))
 (segment (start 34.544 56.134) (end 32.258 56.134) (width 0.381) (layer F.Cu) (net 14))
 (segment (start 36.068 54.102) (end 34.544 56.134) (width 0.381) (layer F.Cu) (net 14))
 (segment (start 38.1 54.102) (end 36.068 54.102) (width 0.381) (layer F.Cu) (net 14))
 (segment (start 38.62 55.13) (end 38.1 54.102) (width 0.381) (layer F.Cu) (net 14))
 (segment (start 40.132 45.708) (end 40.132 48.006) (width 0.381) (layer F.Cu) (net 22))
 (segment (start 45.72 45.466) (end 47.498 43.688) (width 0.381) (layer F.Cu) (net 22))
 (segment (start 45.72 46.99) (end 45.72 45.466) (width 0.381) (layer F.Cu) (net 22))
 (segment (start 43.434 49.276) (end 45.72 46.99) (width 0.381) (layer F.Cu) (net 22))
 (segment (start 41.402 49.276) (end 43.434 49.276) (width 0.381) (layer F.Cu) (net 22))
 (segment (start 40.132 48.006) (end 41.402 49.276) (width 0.381) (layer F.Cu) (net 22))
 (segment (start 47.498 43.688) (end 47.498 43.434) (width 0.381) (layer F.Cu) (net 22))
 (segment (start 38.608 45.454) (end 38.608 47.752) (width 0.381) (layer F.Cu) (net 25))
 (segment (start 41.91 51.054) (end 47.498 51.054) (width 0.381) (layer F.Cu) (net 25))
 (segment (start 38.608 47.752) (end 41.91 51.054) (width 0.381) (layer F.Cu) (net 25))
 (segment (start 36.056 48.768) (end 37.592 48.768) (width 0.381) (layer F.Cu) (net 28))
 (segment (start 37.592 48.768) (end 47.498 58.674) (width 0.381) (layer F.Cu) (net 28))
 (segment (start 44.704 45.708) (end 44.704 45.466) (width 0.381) (layer F.Cu) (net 21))
 (segment (start 44.704 45.466) (end 45.72 44.45) (width 0.381) (layer F.Cu) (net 21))
 (segment (start 45.72 42.672) (end 47.498 40.894) (width 0.381) (layer F.Cu) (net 21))
 (segment (start 45.72 44.45) (end 45.72 42.672) (width 0.381) (layer F.Cu) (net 21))
 (segment (start 44.704 45.708) (end 44.716 45.708) (width 0.381) (layer F.Cu) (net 21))
 (segment (start 34.798 30.48) (end 34.798 34.511) (width 1) (layer F.Cu) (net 5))
 (segment (start 34.798 34.511) (end 35.433 35.146) (width 1) (layer F.Cu) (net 5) (status 20))
 (segment (start 35.433 35.146) (end 36.703 35.146) (width 1) (layer F.Cu) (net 5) (status 30))
 (segment (start 39.878 30.48) (end 39.878 33.241) (width 1) (layer F.Cu) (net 4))
 (segment (start 39.243 33.876) (end 39.243 35.146) (width 1) (layer F.Cu) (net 4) (status 20))
 (segment (start 39.878 33.241) (end 39.243 33.876) (width 1) (layer F.Cu) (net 4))
 (segment (start 39.243 35.146) (end 37.973 35.146) (width 1) (layer F.Cu) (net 4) (status 30))
 (segment (start 44.958 30.48) (end 44.958 30.988) (width 1) (layer F.Cu) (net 33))
 (segment (start 44.958 30.988) (end 42.291 33.655) (width 1) (layer F.Cu) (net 33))
 (segment (start 42.291 33.655) (end 42.291 35.146) (width 1) (layer F.Cu) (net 33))
 (segment (start 42.291 35.146) (end 41.021 35.146) (width 1) (layer F.Cu) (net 33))
 (segment (start 50.038 30.48) (end 47.244 33.274) (width 1) (layer F.Cu) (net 34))
 (segment (start 45.974 33.274) (end 44.831 34.417) (width 1) (layer F.Cu) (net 34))
 (segment (start 47.244 33.274) (end 45.974 33.274) (width 1) (layer F.Cu) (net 34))
 (segment (start 44.831 34.417) (end 44.831 35.146) (width 1) (layer F.Cu) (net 34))
 (segment (start 44.831 35.146) (end 43.561 35.146) (width 1) (layer F.Cu) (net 34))
 (segment (start 37.592 69.85) (end 41.77 69.85) (width 1.6) (layer F.Cu) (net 35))
 (segment (start 41.77 69.85) (end 43.434 71.514) (width 1.6) (layer F.Cu) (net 35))
 (segment (start 34.556 48.768) (end 34.556 46.482) (width 0.381) (layer F.Cu) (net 36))
 (segment (start 34.556 46.482) (end 35.56 45.478) (width 0.381) (layer F.Cu) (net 36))
 (segment (start 35.052 43.93) (end 35.052 44.97) (width 0.381) (layer F.Cu) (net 36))
 (segment (start 35.052 44.97) (end 35.56 45.478) (width 0.381) (layer F.Cu) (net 36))
 (segment (start 37.084 43.954) (end 38.608 43.954) (width 0.381) (layer F.Cu) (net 37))
 (segment (start 38.608 43.954) (end 38.608 43.676) (width 0.381) (layer F.Cu) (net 37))
 (segment (start 38.608 43.676) (end 37.35 42.418) (width 0.381) (layer F.Cu) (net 37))
 (segment (start 40.132 44.208) (end 41.656 44.208) (width 0.381) (layer F.Cu) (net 38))
 (segment (start 41.656 44.208) (end 41.426 44.208) (width 0.381) (layer F.Cu) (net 38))
 (segment (start 41.426 44.208) (end 39.89 42.672) (width 0.381) (layer F.Cu) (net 38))
 (segment (start 44.704 44.208) (end 43.18 44.208) (width 0.381) (layer F.Cu) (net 39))
 (segment (start 43.18 44.208) (end 43.18 44.184) (width 0.381) (layer F.Cu) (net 39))
 (segment (start 43.18 44.184) (end 44.692 42.672) (width 0.381) (layer F.Cu) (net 39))
 (segment (start 44.692 44.196) (end 44.704 44.208) (width 0.381) (layer F.Cu) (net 39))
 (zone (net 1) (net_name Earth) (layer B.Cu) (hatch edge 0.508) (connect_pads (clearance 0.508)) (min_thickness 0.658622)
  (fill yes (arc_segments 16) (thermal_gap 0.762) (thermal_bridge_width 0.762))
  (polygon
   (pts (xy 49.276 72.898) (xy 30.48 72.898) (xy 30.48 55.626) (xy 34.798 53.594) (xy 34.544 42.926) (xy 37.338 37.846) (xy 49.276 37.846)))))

